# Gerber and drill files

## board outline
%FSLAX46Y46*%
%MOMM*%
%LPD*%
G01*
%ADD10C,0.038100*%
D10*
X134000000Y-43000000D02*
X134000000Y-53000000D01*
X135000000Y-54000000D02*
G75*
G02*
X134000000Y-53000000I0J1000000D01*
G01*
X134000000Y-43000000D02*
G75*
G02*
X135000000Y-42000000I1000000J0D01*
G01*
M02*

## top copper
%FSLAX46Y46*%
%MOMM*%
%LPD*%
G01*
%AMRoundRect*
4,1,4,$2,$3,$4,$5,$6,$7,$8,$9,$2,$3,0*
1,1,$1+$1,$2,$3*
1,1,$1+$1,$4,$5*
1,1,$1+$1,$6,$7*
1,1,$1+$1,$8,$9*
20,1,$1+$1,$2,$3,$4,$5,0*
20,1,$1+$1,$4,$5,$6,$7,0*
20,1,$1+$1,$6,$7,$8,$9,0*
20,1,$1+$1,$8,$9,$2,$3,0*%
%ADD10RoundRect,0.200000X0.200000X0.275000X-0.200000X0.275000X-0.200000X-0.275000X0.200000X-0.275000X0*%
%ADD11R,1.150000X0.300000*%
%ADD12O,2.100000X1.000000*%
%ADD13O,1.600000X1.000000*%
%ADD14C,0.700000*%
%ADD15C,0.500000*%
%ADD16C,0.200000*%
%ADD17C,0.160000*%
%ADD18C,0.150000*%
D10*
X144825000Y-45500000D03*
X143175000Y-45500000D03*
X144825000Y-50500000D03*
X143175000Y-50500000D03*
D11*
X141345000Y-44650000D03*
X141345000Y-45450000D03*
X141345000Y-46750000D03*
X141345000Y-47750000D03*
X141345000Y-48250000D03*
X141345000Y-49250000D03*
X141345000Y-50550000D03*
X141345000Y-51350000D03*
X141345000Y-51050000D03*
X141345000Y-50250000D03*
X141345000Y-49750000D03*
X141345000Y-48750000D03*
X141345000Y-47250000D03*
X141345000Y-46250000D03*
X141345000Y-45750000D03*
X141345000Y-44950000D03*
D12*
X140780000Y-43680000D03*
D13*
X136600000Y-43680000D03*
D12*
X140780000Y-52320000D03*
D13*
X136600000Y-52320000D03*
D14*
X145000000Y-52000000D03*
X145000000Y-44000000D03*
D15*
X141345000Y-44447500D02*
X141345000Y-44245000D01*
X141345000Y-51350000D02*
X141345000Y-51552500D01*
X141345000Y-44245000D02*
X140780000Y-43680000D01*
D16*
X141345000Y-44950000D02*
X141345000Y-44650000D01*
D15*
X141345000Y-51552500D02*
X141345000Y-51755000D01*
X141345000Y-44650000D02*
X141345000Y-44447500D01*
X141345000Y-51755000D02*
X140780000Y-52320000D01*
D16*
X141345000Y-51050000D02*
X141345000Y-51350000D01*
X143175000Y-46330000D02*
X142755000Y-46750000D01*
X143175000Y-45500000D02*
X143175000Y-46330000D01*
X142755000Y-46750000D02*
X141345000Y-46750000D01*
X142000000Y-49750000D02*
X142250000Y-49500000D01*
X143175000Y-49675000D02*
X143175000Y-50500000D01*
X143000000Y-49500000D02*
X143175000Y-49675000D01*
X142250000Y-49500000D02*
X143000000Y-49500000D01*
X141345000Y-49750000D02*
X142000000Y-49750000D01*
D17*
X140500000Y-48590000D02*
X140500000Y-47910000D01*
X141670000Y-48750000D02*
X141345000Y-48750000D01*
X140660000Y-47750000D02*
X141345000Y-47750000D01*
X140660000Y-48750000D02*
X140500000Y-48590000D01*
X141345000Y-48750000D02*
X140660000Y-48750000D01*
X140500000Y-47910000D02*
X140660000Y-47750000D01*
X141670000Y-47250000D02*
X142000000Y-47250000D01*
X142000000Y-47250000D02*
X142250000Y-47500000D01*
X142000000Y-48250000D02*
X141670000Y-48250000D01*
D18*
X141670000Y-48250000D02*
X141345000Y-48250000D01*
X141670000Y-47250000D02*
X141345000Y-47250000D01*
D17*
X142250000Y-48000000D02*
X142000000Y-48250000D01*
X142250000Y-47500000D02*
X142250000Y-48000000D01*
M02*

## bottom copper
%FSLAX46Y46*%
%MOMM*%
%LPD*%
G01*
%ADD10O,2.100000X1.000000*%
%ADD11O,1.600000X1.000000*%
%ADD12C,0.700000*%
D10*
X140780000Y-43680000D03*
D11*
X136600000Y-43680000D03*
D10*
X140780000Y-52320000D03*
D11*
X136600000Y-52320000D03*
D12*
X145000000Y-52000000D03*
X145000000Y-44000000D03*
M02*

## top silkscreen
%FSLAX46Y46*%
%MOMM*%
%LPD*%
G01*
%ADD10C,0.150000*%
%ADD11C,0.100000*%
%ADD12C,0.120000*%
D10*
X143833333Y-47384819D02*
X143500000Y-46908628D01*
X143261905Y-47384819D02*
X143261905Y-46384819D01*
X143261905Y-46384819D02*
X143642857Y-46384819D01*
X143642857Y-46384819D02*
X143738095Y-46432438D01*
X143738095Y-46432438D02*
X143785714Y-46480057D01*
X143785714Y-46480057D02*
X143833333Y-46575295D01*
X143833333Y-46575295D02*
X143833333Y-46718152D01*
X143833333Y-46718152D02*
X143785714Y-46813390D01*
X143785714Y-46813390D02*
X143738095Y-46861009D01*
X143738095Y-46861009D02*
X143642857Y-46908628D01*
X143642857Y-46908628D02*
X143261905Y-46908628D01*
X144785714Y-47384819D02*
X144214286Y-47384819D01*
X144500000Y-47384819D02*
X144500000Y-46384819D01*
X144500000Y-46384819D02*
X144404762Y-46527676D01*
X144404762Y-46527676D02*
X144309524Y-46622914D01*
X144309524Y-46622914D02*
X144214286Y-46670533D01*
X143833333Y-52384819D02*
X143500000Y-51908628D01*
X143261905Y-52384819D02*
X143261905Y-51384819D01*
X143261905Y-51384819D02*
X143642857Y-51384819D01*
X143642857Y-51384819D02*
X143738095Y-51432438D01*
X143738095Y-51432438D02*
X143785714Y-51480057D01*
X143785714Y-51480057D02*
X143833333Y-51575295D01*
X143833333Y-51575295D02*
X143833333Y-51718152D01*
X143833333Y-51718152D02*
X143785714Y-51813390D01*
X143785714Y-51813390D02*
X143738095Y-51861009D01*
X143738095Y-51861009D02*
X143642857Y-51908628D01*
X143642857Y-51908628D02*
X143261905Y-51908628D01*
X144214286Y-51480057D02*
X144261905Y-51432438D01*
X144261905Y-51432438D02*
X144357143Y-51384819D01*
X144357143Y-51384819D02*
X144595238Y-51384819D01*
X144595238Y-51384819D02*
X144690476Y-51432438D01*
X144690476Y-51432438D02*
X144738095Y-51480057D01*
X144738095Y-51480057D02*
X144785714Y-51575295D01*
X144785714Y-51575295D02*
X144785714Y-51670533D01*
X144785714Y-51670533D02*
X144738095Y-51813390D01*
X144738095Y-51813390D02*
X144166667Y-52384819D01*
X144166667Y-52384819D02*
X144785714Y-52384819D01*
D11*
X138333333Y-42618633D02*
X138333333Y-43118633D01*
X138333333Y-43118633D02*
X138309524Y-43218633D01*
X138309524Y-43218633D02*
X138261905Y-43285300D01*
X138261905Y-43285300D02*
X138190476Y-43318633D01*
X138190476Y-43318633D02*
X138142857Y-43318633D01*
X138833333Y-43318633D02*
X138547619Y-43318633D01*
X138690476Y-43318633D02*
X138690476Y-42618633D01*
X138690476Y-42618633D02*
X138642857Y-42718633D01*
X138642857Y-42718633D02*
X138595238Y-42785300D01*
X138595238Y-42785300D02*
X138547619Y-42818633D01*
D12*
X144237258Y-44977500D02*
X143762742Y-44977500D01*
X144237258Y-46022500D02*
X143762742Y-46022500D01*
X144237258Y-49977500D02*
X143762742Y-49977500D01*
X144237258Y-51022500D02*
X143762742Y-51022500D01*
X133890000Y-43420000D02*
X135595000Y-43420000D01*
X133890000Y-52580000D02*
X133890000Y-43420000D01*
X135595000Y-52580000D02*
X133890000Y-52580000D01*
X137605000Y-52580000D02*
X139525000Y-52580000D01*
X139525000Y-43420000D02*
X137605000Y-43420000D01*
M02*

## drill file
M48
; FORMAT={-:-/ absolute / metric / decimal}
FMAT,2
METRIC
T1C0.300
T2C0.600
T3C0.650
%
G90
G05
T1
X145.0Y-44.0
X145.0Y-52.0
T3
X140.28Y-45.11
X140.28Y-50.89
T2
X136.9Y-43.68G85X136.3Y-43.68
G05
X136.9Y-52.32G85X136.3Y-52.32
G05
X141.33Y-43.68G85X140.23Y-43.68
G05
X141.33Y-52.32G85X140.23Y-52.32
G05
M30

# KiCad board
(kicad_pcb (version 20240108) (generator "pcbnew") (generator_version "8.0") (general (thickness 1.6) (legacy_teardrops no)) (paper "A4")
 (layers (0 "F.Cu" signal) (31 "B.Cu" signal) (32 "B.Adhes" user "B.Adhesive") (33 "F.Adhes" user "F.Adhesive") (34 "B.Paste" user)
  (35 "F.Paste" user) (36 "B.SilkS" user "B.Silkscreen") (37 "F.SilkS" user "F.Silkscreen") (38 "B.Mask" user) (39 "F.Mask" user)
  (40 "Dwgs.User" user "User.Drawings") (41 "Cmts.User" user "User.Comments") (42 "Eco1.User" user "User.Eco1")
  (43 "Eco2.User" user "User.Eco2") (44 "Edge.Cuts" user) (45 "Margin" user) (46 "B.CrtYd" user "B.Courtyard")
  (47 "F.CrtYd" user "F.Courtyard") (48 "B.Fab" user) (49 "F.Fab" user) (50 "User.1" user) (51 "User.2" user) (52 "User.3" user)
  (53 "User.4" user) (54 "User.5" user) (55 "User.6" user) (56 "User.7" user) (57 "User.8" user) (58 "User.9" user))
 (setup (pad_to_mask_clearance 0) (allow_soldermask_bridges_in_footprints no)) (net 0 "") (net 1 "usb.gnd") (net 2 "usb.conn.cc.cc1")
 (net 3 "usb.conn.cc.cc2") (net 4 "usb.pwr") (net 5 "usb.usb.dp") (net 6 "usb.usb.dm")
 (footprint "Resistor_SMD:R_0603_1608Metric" (layer "F.Cu") (at 144 45.5 180)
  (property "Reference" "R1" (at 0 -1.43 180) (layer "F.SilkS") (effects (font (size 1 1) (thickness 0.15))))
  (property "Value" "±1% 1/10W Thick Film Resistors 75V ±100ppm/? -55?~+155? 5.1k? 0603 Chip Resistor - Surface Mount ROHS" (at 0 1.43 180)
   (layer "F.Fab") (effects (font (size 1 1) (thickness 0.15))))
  (fp_line (start -0.237258 0.5225) (end 0.237258 0.5225) (stroke (width 0.12) (type solid)) (layer "F.SilkS"))
  (fp_line (start -0.237258 -0.5225) (end 0.237258 -0.5225) (stroke (width 0.12) (type solid)) (layer "F.SilkS"))
  (pad "1" smd roundrect (at -0.825 0 180) (size 0.8 0.95) (layers "F.Cu" "F.Paste" "F.Mask") (roundrect_rratio 0.25) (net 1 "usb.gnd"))
  (pad "2" smd roundrect (at 0.825 0 180) (size 0.8 0.95) (layers "F.Cu" "F.Paste" "F.Mask") (roundrect_rratio 0.25)
   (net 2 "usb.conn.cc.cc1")))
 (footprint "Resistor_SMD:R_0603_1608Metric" (layer "F.Cu") (at 144 50.5 180)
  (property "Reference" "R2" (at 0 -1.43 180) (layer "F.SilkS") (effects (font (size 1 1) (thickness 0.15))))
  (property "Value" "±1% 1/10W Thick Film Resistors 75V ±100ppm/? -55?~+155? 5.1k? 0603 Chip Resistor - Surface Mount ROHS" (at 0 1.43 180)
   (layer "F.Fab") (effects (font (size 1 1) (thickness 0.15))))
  (fp_line (start -0.237258 0.5225) (end 0.237258 0.5225) (stroke (width 0.12) (type solid)) (layer "F.SilkS"))
  (fp_line (start -0.237258 -0.5225) (end 0.237258 -0.5225) (stroke (width 0.12) (type solid)) (layer "F.SilkS"))
  (pad "1" smd roundrect (at -0.825 0 180) (size 0.8 0.95) (layers "F.Cu" "F.Paste" "F.Mask") (roundrect_rratio 0.25) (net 1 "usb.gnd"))
  (pad "2" smd roundrect (at 0.825 0 180) (size 0.8 0.95) (layers "F.Cu" "F.Paste" "F.Mask") (roundrect_rratio 0.25)
   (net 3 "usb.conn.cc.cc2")))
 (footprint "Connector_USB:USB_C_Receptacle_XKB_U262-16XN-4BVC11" (layer "F.Cu") (at 137.675 48 -90)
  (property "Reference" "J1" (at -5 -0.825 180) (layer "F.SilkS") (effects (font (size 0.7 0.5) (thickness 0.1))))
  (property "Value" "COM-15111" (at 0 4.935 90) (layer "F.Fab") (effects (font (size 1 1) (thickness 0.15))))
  (fp_line (start -4.58 3.785) (end -4.58 2.08) (stroke (width 0.12) (type solid)) (layer "F.SilkS"))
  (fp_line (start 4.58 3.785) (end -4.58 3.785) (stroke (width 0.12) (type solid)) (layer "F.SilkS"))
  (fp_line (start 4.58 2.08) (end 4.58 3.785) (stroke (width 0.12) (type solid)) (layer "F.SilkS"))
  (fp_line (start 4.58 0.07) (end 4.58 -1.85) (stroke (width 0.12) (type solid)) (layer "F.SilkS"))
  (fp_line (start -4.58 -1.85) (end -4.58 0.07) (stroke (width 0.12) (type solid)) (layer "F.SilkS"))
  (pad "" np_thru_hole circle (at -2.89 -2.605 270) (size 0.65 0.65) (drill 0.65) (layers "*.Cu" "*.Mask"))
  (pad "" np_thru_hole circle (at 2.89 -2.605 270) (size 0.65 0.65) (drill 0.65) (layers "*.Cu" "*.Mask"))
  (pad "A1" smd rect (at -3.35 -3.67 270) (size 0.3 1.15) (layers "F.Cu" "F.Paste" "F.Mask") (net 1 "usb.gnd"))
  (pad "A4" smd rect (at -2.55 -3.67 270) (size 0.3 1.15) (layers "F.Cu" "F.Paste" "F.Mask") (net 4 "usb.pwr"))
  (pad "A5" smd rect (at -1.25 -3.67 270) (size 0.3 1.15) (layers "F.Cu" "F.Paste" "F.Mask") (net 2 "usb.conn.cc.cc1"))
  (pad "A6" smd rect (at -0.25 -3.67 270) (size 0.3 1.15) (layers "F.Cu" "F.Paste" "F.Mask") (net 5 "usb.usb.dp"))
  (pad "A7" smd rect (at 0.25 -3.67 270) (size 0.3 1.15) (layers "F.Cu" "F.Paste" "F.Mask") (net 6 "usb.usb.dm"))
  (pad "A8" smd rect (at 1.25 -3.67 270) (size 0.3 1.15) (layers "F.Cu" "F.Paste" "F.Mask"))
  (pad "A9" smd rect (at 2.55 -3.67 270) (size 0.3 1.15) (layers "F.Cu" "F.Paste" "F.Mask") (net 4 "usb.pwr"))
  (pad "A12" smd rect (at 3.35 -3.67 270) (size 0.3 1.15) (layers "F.Cu" "F.Paste" "F.Mask") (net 1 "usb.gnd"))
  (pad "B1" smd rect (at 3.05 -3.67 270) (size 0.3 1.15) (layers "F.Cu" "F.Paste" "F.Mask") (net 1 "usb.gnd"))
  (pad "B4" smd rect (at 2.25 -3.67 270) (size 0.3 1.15) (layers "F.Cu" "F.Paste" "F.Mask") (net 4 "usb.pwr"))
  (pad "B5" smd rect (at 1.75 -3.67 270) (size 0.3 1.15) (layers "F.Cu" "F.Paste" "F.Mask") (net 3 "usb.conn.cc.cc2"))
  (pad "B6" smd rect (at 0.75 -3.67 270) (size 0.3 1.15) (layers "F.Cu" "F.Paste" "F.Mask") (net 5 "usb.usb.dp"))
  (pad "B7" smd rect (at -0.75 -3.67 270) (size 0.3 1.15) (layers "F.Cu" "F.Paste" "F.Mask") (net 6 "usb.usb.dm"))
  (pad "B8" smd rect (at -1.75 -3.67 270) (size 0.3 1.15) (layers "F.Cu" "F.Paste" "F.Mask"))
  (pad "B9" smd rect (at -2.25 -3.67 270) (size 0.3 1.15) (layers "F.Cu" "F.Paste" "F.Mask") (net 4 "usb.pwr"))
  (pad "B12" smd rect (at -3.05 -3.67 270) (size 0.3 1.15) (layers "F.Cu" "F.Paste" "F.Mask") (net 1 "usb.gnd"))
  (pad "S1" thru_hole oval (at -4.32 -3.105 270) (size 1 2.1) (drill oval 0.6 1.7) (layers "*.Cu" "*.Mask") (remove_unused_layers no)
   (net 1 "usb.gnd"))
  (pad "S1" thru_hole oval (at -4.32 1.075 270) (size 1 1.6) (drill oval 0.6 1.2) (layers "*.Cu" "*.Mask") (remove_unused_layers no)
   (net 1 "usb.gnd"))
  (pad "S1" thru_hole oval (at 4.32 -3.105 270) (size 1 2.1) (drill oval 0.6 1.7) (layers "*.Cu" "*.Mask") (remove_unused_layers no)
   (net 1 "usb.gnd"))
  (pad "S1" thru_hole oval (at 4.32 1.075 270) (size 1 1.6) (drill oval 0.6 1.2) (layers "*.Cu" "*.Mask") (remove_unused_layers no)
   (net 1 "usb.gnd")))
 (gr_line (start 134 43) (end 134 53) (stroke (width 0.0381) (type solid)) (layer "Edge.Cuts"))
 (gr_arc (start 135 54) (mid 134.292893 53.707107) (end 134 53) (stroke (width 0.0381) (type solid)) (layer "Edge.Cuts"))
 (gr_arc (start 134 43) (mid 134.292893 42.292893) (end 135 42) (stroke (width 0.0381) (type solid)) (layer "Edge.Cuts"))
 (segment (start 141.345 44.4475) (end 141.345 44.245) (width 0.5) (layer "F.Cu") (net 1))
 (segment (start 141.345 51.35) (end 141.345 51.5525) (width 0.5) (layer "F.Cu") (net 1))
 (segment (start 141.345 44.245) (end 140.78 43.68) (width 0.5) (layer "F.Cu") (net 1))
 (segment (start 141.345 44.95) (end 141.345 44.65) (width 0.2) (layer "F.Cu") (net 1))
 (segment (start 141.345 51.5525) (end 141.345 51.755) (width 0.5) (layer "F.Cu") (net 1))
 (segment (start 141.345 44.65) (end 141.345 44.4475) (width 0.5) (layer "F.Cu") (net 1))
 (segment (start 141.345 51.755) (end 140.78 52.32) (width 0.5) (layer "F.Cu") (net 1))
 (segment (start 141.345 51.05) (end 141.345 51.35) (width 0.2) (layer "F.Cu") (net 1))
 (via (at 145 52) (size 0.7) (drill 0.3) (layers "F.Cu" "B.Cu") (free yes) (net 1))
 (via (at 145 44) (size 0.7) (drill 0.3) (layers "F.Cu" "B.Cu") (free yes) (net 1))
 (segment (start 143.175 46.33) (end 142.755 46.75) (width 0.2) (layer "F.Cu") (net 2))
 (segment (start 143.175 45.5) (end 143.175 46.33) (width 0.2) (layer "F.Cu") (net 2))
 (segment (start 142.755 46.75) (end 141.345 46.75) (width 0.2) (layer "F.Cu") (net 2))
 (segment (start 142 49.75) (end 142.25 49.5) (width 0.2) (layer "F.Cu") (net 3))
 (segment (start 143.175 49.675) (end 143.175 50.5) (width 0.2) (layer "F.Cu") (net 3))
 (segment (start 143 49.5) (end 143.175 49.675) (width 0.2) (layer "F.Cu") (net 3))
 (segment (start 142.25 49.5) (end 143 49.5) (width 0.2) (layer "F.Cu") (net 3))
 (segment (start 141.345 49.75) (end 142 49.75) (width 0.2) (layer "F.Cu") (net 3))
 (segment (start 140.5 48.59) (end 140.5 47.91) (width 0.16) (layer "F.Cu") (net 5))
 (segment (start 141.67 48.75) (end 141.345 48.75) (width 0.16) (layer "F.Cu") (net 5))
 (segment (start 140.66 47.75) (end 141.345 47.75) (width 0.16) (layer "F.Cu") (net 5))
 (segment (start 140.66 48.75) (end 140.5 48.59) (width 0.16) (layer "F.Cu") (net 5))
 (segment (start 141.345 48.75) (end 140.66 48.75) (width 0.16) (layer "F.Cu") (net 5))
 (segment (start 140.5 47.91) (end 140.66 47.75) (width 0.16) (layer "F.Cu") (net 5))
 (segment (start 141.67 47.25) (end 142 47.25) (width 0.16) (layer "F.Cu") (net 6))
 (segment (start 142 47.25) (end 142.25 47.5) (width 0.16) (layer "F.Cu") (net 6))
 (segment (start 142 48.25) (end 141.67 48.25) (width 0.16) (layer "F.Cu") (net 6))
 (segment (start 141.67 48.25) (end 141.345 48.25) (width 0.15) (layer "F.Cu") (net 6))
 (segment (start 141.67 47.25) (end 141.345 47.25) (width 0.15) (layer "F.Cu") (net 6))
 (segment (start 142.25 48) (end 142 48.25) (width 0.16) (layer "F.Cu") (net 6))
 (segment (start 142.25 47.5) (end 142.25 48) (width 0.16) (layer "F.Cu") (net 6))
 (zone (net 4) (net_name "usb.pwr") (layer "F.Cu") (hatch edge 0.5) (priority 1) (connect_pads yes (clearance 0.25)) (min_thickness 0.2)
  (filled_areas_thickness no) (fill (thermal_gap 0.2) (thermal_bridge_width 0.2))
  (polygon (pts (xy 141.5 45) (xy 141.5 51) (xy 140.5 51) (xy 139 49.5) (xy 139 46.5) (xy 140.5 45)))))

